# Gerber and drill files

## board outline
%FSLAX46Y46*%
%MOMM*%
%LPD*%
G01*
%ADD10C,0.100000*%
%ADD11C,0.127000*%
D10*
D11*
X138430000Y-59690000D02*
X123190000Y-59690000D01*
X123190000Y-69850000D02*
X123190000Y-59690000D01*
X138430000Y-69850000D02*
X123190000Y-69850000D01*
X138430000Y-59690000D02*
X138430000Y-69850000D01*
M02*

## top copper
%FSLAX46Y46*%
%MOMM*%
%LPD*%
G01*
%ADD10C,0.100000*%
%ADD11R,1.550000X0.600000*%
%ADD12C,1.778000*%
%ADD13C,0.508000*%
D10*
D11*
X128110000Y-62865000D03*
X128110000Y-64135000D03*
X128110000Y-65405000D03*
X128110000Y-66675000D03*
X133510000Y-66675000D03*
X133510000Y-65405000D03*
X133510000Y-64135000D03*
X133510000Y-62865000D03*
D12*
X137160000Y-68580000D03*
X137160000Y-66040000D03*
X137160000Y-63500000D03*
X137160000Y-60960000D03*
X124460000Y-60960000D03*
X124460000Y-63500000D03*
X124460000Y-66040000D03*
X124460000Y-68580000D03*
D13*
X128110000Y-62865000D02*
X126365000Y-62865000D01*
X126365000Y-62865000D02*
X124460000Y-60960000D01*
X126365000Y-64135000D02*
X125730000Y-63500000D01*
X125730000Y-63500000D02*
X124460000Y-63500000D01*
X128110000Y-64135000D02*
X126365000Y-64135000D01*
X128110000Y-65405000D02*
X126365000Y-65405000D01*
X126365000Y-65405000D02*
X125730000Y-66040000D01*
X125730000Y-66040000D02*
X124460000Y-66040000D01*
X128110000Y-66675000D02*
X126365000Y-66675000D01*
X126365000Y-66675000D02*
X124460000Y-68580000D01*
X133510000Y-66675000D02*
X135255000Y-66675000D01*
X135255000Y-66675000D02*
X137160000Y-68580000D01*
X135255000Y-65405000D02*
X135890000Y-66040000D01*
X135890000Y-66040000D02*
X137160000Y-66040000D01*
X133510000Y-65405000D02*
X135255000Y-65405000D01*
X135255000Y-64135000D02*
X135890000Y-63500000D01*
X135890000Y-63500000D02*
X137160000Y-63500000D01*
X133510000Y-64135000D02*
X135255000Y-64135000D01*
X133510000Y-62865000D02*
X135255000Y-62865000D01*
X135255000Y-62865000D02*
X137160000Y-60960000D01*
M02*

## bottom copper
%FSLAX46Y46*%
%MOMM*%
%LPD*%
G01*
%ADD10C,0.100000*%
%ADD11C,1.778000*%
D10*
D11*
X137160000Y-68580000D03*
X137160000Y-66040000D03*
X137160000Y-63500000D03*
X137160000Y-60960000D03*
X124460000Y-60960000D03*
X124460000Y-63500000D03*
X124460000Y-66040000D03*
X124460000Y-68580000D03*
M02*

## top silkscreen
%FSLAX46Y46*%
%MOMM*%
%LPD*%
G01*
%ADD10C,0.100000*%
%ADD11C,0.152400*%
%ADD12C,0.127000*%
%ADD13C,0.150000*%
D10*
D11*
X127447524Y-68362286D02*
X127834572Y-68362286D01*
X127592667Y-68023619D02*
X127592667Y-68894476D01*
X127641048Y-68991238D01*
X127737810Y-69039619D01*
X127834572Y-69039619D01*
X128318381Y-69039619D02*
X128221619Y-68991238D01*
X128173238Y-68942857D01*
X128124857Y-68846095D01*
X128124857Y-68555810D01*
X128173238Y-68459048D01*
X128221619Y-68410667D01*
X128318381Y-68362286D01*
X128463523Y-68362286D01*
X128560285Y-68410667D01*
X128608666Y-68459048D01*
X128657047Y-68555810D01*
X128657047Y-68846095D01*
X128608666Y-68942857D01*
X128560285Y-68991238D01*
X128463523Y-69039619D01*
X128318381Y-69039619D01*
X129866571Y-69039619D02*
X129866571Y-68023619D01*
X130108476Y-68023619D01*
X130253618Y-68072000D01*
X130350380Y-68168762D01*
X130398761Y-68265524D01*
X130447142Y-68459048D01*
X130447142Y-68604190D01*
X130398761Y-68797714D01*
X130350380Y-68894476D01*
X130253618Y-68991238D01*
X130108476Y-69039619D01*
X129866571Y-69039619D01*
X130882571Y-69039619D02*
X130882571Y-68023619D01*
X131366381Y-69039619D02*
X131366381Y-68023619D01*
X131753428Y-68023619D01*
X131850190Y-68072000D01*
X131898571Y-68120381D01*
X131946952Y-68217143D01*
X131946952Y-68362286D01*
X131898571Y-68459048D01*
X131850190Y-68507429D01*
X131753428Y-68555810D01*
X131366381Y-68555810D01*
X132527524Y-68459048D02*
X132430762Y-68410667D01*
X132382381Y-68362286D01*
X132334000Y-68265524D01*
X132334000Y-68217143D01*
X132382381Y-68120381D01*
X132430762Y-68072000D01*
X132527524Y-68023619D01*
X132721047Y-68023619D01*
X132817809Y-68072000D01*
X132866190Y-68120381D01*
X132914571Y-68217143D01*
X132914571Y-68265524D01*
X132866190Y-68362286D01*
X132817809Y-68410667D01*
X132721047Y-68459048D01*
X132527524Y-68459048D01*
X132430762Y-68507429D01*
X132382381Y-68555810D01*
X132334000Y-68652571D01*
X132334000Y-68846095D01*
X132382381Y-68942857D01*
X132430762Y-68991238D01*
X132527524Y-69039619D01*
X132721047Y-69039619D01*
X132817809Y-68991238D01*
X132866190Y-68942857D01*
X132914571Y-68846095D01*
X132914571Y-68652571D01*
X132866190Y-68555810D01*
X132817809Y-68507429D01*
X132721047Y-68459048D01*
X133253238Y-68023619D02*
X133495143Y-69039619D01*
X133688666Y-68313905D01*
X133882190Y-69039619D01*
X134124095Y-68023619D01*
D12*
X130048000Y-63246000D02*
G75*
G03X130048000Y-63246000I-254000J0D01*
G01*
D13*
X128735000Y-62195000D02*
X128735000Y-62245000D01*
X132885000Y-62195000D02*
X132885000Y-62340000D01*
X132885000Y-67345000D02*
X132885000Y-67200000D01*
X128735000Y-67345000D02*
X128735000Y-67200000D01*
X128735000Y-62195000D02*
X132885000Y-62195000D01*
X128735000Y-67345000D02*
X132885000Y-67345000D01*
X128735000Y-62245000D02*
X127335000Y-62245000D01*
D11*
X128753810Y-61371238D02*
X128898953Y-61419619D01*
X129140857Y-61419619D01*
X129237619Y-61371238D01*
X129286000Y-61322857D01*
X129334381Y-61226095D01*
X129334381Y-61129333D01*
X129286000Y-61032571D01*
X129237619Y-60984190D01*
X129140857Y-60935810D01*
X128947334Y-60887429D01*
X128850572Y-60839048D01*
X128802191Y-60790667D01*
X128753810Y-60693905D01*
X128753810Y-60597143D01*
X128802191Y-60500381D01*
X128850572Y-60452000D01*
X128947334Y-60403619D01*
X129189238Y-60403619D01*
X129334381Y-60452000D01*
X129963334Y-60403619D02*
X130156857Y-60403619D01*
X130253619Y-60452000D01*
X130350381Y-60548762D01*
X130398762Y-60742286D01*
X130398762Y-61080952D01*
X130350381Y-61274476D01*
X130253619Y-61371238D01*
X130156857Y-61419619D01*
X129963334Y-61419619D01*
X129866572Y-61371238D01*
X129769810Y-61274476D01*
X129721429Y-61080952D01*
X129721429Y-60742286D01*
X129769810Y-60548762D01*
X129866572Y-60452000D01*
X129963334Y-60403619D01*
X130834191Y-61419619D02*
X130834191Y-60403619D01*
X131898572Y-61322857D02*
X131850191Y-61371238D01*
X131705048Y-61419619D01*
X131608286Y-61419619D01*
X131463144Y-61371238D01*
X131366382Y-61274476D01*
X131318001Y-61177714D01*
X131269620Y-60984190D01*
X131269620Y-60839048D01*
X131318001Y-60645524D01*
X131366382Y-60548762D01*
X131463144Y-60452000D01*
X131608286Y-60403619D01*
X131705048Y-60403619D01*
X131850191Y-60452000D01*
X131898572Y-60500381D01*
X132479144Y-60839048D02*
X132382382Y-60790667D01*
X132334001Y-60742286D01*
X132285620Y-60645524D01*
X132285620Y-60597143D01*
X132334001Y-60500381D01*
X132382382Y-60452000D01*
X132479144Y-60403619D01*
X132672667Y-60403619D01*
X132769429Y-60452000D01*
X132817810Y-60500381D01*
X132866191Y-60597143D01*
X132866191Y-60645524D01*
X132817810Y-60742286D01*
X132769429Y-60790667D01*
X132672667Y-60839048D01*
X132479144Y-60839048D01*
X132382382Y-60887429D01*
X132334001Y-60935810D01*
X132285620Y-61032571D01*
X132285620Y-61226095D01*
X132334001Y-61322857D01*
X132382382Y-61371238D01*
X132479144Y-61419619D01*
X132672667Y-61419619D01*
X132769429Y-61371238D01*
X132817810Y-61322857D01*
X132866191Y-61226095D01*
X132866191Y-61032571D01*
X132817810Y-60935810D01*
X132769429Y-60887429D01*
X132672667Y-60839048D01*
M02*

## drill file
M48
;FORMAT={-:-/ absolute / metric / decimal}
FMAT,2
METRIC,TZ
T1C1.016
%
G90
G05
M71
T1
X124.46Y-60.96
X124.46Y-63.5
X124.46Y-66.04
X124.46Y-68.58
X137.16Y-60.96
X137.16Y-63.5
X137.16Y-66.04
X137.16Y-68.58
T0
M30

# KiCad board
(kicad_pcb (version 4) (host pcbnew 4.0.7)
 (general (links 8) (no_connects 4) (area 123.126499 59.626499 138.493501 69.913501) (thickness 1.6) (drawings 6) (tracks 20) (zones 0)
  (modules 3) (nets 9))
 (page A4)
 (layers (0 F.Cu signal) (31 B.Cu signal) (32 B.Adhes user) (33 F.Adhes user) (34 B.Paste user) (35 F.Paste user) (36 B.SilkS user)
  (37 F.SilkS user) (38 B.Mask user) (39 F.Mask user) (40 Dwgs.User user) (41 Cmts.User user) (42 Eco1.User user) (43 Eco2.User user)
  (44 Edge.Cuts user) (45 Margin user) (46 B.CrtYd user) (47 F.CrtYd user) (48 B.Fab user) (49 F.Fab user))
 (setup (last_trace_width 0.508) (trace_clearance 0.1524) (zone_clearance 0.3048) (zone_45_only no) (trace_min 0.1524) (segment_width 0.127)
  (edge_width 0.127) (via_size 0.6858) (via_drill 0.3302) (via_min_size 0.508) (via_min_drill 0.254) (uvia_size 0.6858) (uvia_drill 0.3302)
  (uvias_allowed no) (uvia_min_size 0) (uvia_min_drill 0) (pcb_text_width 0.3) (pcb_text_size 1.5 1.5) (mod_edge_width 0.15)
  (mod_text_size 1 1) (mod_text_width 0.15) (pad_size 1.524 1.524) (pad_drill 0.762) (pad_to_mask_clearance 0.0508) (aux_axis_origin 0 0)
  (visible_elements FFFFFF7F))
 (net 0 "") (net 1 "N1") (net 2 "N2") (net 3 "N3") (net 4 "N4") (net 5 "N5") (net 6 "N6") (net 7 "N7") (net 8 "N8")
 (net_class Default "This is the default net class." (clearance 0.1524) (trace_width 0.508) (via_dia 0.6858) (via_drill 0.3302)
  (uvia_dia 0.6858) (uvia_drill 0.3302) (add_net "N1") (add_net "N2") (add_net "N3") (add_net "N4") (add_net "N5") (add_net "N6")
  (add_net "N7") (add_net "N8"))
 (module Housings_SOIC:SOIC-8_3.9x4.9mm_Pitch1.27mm (layer F.Cu) (at 130.81 64.77)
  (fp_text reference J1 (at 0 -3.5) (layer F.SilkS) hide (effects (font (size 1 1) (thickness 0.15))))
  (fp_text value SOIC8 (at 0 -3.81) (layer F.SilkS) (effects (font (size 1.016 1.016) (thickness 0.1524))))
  (fp_line (start -2.075 -2.575) (end -2.075 -2.525) (layer F.SilkS) (width 0.15))
  (fp_line (start 2.075 -2.575) (end 2.075 -2.43) (layer F.SilkS) (width 0.15))
  (fp_line (start 2.075 2.575) (end 2.075 2.43) (layer F.SilkS) (width 0.15))
  (fp_line (start -2.075 2.575) (end -2.075 2.43) (layer F.SilkS) (width 0.15))
  (fp_line (start -2.075 -2.575) (end 2.075 -2.575) (layer F.SilkS) (width 0.15))
  (fp_line (start -2.075 2.575) (end 2.075 2.575) (layer F.SilkS) (width 0.15))
  (fp_line (start -2.075 -2.525) (end -3.475 -2.525) (layer F.SilkS) (width 0.15))
  (pad 1 smd rect (at -2.7 -1.905) (size 1.55 0.6) (layers F.Cu F.Paste F.Mask) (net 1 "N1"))
  (pad 2 smd rect (at -2.7 -0.635) (size 1.55 0.6) (layers F.Cu F.Paste F.Mask) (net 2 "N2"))
  (pad 3 smd rect (at -2.7 0.635) (size 1.55 0.6) (layers F.Cu F.Paste F.Mask) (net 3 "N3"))
  (pad 4 smd rect (at -2.7 1.905) (size 1.55 0.6) (layers F.Cu F.Paste F.Mask) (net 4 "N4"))
  (pad 5 smd rect (at 2.7 1.905) (size 1.55 0.6) (layers F.Cu F.Paste F.Mask) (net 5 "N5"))
  (pad 6 smd rect (at 2.7 0.635) (size 1.55 0.6) (layers F.Cu F.Paste F.Mask) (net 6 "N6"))
  (pad 7 smd rect (at 2.7 -0.635) (size 1.55 0.6) (layers F.Cu F.Paste F.Mask) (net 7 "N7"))
  (pad 8 smd rect (at 2.7 -1.905) (size 1.55 0.6) (layers F.Cu F.Paste F.Mask) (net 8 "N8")))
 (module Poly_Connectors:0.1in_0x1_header (layer B.Cu) (at 137.16 68.58 180)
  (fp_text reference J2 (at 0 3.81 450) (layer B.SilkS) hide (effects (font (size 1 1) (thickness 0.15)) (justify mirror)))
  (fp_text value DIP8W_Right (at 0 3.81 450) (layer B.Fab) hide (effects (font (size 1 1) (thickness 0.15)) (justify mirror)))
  (pad 1 thru_hole circle (at 0 0 180) (size 1.778 1.778) (drill 1.016) (layers *.Cu *.Mask) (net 5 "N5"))
  (pad 2 thru_hole circle (at 0 2.54 180) (size 1.778 1.778) (drill 1.016) (layers *.Cu *.Mask) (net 6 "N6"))
  (pad 3 thru_hole circle (at 0 5.08 180) (size 1.778 1.778) (drill 1.016) (layers *.Cu *.Mask) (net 7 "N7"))
  (pad 4 thru_hole circle (at 0 7.62 180) (size 1.778 1.778) (drill 1.016) (layers *.Cu *.Mask) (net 8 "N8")))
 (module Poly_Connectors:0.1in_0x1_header (layer B.Cu) (at 124.46 60.96)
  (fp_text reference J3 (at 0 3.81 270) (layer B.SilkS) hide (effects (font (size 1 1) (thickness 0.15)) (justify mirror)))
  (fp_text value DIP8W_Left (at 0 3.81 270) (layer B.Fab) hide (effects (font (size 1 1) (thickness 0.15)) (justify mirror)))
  (pad 1 thru_hole circle (at 0 0) (size 1.778 1.778) (drill 1.016) (layers *.Cu *.Mask) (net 1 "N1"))
  (pad 2 thru_hole circle (at 0 2.54) (size 1.778 1.778) (drill 1.016) (layers *.Cu *.Mask) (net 2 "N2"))
  (pad 3 thru_hole circle (at 0 5.08) (size 1.778 1.778) (drill 1.016) (layers *.Cu *.Mask) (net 3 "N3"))
  (pad 4 thru_hole circle (at 0 7.62) (size 1.778 1.778) (drill 1.016) (layers *.Cu *.Mask) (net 4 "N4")))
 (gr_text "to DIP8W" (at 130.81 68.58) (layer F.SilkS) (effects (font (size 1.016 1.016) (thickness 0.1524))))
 (gr_circle (center 129.794 63.246) (end 129.794 62.992) (layer F.SilkS) (width 0.127))
 (gr_line (start 138.43 59.69) (end 123.19 59.69) (layer Edge.Cuts) (width 0.127))
 (gr_line (start 123.19 69.85) (end 123.19 59.69) (layer Edge.Cuts) (width 0.127))
 (gr_line (start 138.43 69.85) (end 123.19 69.85) (layer Edge.Cuts) (width 0.127))
 (gr_line (start 138.43 59.69) (end 138.43 69.85) (layer Edge.Cuts) (width 0.127))
 (segment (start 128.11 62.865) (end 126.365 62.865) (width 0.508) (layer F.Cu) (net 1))
 (segment (start 126.365 62.865) (end 124.46 60.96) (width 0.508) (layer F.Cu) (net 1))
 (segment (start 126.365 64.135) (end 125.73 63.5) (width 0.508) (layer F.Cu) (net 2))
 (segment (start 125.73 63.5) (end 124.46 63.5) (width 0.508) (layer F.Cu) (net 2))
 (segment (start 128.11 64.135) (end 126.365 64.135) (width 0.508) (layer F.Cu) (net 2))
 (segment (start 128.11 65.405) (end 126.365 65.405) (width 0.508) (layer F.Cu) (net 3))
 (segment (start 126.365 65.405) (end 125.73 66.04) (width 0.508) (layer F.Cu) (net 3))
 (segment (start 125.73 66.04) (end 124.46 66.04) (width 0.508) (layer F.Cu) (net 3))
 (segment (start 128.11 66.675) (end 126.365 66.675) (width 0.508) (layer F.Cu) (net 4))
 (segment (start 126.365 66.675) (end 124.46 68.58) (width 0.508) (layer F.Cu) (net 4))
 (segment (start 133.51 66.675) (end 135.255 66.675) (width 0.508) (layer F.Cu) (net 5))
 (segment (start 135.255 66.675) (end 137.16 68.58) (width 0.508) (layer F.Cu) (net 5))
 (segment (start 135.255 65.405) (end 135.89 66.04) (width 0.508) (layer F.Cu) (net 6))
 (segment (start 135.89 66.04) (end 137.16 66.04) (width 0.508) (layer F.Cu) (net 6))
 (segment (start 133.51 65.405) (end 135.255 65.405) (width 0.508) (layer F.Cu) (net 6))
 (segment (start 135.255 64.135) (end 135.89 63.5) (width 0.508) (layer F.Cu) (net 7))
 (segment (start 135.89 63.5) (end 137.16 63.5) (width 0.508) (layer F.Cu) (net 7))
 (segment (start 133.51 64.135) (end 135.255 64.135) (width 0.508) (layer F.Cu) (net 7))
 (segment (start 133.51 62.865) (end 135.255 62.865) (width 0.508) (layer F.Cu) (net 8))
 (segment (start 135.255 62.865) (end 137.16 60.96) (width 0.508) (layer F.Cu) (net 8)))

